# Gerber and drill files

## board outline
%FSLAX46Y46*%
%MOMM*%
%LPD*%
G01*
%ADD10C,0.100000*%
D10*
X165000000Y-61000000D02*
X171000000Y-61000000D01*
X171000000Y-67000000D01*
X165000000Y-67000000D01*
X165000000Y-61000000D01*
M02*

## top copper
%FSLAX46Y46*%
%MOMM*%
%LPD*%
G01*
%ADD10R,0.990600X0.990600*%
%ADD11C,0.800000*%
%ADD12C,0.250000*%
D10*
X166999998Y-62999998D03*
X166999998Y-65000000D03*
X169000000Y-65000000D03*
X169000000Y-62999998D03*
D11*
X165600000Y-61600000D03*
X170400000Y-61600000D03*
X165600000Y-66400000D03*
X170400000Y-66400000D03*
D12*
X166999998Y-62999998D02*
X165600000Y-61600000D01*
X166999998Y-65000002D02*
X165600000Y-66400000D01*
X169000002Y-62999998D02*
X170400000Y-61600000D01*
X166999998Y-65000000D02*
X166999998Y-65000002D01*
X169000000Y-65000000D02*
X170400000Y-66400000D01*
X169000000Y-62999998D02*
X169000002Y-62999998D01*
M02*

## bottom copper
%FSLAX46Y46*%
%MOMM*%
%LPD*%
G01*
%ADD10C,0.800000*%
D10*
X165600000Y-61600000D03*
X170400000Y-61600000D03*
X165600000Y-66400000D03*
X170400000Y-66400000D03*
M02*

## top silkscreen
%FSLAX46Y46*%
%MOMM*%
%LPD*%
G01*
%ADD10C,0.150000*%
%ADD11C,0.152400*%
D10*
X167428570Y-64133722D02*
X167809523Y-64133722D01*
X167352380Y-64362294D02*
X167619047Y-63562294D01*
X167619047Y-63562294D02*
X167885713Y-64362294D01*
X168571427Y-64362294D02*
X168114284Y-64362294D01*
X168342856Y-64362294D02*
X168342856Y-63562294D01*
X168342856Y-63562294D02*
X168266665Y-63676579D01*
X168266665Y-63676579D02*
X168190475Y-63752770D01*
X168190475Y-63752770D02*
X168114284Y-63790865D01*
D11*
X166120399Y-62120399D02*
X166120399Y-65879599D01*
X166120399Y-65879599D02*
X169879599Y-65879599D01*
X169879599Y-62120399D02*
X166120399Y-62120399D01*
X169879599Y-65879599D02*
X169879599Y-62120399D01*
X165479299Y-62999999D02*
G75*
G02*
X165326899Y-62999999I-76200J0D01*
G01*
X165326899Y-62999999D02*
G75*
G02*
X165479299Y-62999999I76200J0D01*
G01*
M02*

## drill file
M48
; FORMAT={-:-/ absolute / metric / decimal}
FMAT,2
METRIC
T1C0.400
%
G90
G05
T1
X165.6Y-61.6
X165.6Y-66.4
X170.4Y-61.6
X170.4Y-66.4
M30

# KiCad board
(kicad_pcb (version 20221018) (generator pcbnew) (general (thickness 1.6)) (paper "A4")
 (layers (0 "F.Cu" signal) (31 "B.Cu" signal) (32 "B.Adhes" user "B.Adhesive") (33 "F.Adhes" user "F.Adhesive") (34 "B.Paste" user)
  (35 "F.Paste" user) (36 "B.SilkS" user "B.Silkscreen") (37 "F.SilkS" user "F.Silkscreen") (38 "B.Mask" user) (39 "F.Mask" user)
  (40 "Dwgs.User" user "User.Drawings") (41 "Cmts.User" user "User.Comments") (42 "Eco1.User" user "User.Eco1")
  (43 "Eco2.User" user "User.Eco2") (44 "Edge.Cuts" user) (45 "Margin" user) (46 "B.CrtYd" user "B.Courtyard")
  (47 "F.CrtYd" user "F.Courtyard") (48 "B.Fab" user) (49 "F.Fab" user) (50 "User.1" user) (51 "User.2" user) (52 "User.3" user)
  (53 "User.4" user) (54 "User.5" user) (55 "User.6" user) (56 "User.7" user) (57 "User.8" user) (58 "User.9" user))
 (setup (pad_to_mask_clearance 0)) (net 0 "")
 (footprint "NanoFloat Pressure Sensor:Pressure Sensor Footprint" (layer "F.Cu") (at 167.999999 63.999999)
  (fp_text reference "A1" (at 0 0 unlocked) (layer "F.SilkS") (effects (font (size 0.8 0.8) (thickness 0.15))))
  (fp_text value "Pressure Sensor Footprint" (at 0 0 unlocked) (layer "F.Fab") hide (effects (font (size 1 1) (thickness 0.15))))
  (fp_line (start -1.8796 -1.8796) (end -1.8796 1.8796) (stroke (width 0.1524) (type solid)) (layer "F.SilkS"))
  (fp_line (start -1.8796 1.8796) (end 1.8796 1.8796) (stroke (width 0.1524) (type solid)) (layer "F.SilkS"))
  (fp_line (start 1.8796 -1.8796) (end -1.8796 -1.8796) (stroke (width 0.1524) (type solid)) (layer "F.SilkS"))
  (fp_line (start 1.8796 1.8796) (end 1.8796 -1.8796) (stroke (width 0.1524) (type solid)) (layer "F.SilkS"))
  (fp_circle (center -2.5969 -1) (end -2.5207 -1) (stroke (width 0.1524) (type solid)) (fill none) (layer "F.SilkS"))
  (pad "1" smd rect (at -1.000001 -1.000001) (size 0.9906 0.9906) (layers "F.Cu" "F.Paste" "F.Mask"))
  (pad "2" smd rect (at -1.000001 1.000001) (size 0.9906 0.9906) (layers "F.Cu" "F.Paste" "F.Mask"))
  (pad "3" smd rect (at 1.000001 1.000001) (size 0.9906 0.9906) (layers "F.Cu" "F.Paste" "F.Mask"))
  (pad "4" smd rect (at 1.000001 -1.000001) (size 0.9906 0.9906) (layers "F.Cu" "F.Paste" "F.Mask")))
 (gr_rect (start 165 61) (end 171 67) (stroke (width 0.1) (type default)) (fill none) (layer "Edge.Cuts"))
 (segment (start 166.999998 62.999998) (end 165.6 61.6) (width 0.25) (layer "F.Cu") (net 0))
 (segment (start 166.999998 65.000002) (end 165.6 66.4) (width 0.25) (layer "F.Cu") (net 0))
 (segment (start 169.000002 62.999998) (end 170.4 61.6) (width 0.25) (layer "F.Cu") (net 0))
 (segment (start 166.999998 65) (end 166.999998 65.000002) (width 0.25) (layer "F.Cu") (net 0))
 (segment (start 169 65) (end 170.4 66.4) (width 0.25) (layer "F.Cu") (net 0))
 (segment (start 169 62.999998) (end 169.000002 62.999998) (width 0.25) (layer "F.Cu") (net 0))
 (via (at 165.6 61.6) (size 0.8) (drill 0.4) (layers "F.Cu" "B.Cu") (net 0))
 (via (at 170.4 61.6) (size 0.8) (drill 0.4) (layers "F.Cu" "B.Cu") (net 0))
 (via (at 165.6 66.4) (size 0.8) (drill 0.4) (layers "F.Cu" "B.Cu") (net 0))
 (via (at 170.4 66.4) (size 0.8) (drill 0.4) (layers "F.Cu" "B.Cu") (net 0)))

